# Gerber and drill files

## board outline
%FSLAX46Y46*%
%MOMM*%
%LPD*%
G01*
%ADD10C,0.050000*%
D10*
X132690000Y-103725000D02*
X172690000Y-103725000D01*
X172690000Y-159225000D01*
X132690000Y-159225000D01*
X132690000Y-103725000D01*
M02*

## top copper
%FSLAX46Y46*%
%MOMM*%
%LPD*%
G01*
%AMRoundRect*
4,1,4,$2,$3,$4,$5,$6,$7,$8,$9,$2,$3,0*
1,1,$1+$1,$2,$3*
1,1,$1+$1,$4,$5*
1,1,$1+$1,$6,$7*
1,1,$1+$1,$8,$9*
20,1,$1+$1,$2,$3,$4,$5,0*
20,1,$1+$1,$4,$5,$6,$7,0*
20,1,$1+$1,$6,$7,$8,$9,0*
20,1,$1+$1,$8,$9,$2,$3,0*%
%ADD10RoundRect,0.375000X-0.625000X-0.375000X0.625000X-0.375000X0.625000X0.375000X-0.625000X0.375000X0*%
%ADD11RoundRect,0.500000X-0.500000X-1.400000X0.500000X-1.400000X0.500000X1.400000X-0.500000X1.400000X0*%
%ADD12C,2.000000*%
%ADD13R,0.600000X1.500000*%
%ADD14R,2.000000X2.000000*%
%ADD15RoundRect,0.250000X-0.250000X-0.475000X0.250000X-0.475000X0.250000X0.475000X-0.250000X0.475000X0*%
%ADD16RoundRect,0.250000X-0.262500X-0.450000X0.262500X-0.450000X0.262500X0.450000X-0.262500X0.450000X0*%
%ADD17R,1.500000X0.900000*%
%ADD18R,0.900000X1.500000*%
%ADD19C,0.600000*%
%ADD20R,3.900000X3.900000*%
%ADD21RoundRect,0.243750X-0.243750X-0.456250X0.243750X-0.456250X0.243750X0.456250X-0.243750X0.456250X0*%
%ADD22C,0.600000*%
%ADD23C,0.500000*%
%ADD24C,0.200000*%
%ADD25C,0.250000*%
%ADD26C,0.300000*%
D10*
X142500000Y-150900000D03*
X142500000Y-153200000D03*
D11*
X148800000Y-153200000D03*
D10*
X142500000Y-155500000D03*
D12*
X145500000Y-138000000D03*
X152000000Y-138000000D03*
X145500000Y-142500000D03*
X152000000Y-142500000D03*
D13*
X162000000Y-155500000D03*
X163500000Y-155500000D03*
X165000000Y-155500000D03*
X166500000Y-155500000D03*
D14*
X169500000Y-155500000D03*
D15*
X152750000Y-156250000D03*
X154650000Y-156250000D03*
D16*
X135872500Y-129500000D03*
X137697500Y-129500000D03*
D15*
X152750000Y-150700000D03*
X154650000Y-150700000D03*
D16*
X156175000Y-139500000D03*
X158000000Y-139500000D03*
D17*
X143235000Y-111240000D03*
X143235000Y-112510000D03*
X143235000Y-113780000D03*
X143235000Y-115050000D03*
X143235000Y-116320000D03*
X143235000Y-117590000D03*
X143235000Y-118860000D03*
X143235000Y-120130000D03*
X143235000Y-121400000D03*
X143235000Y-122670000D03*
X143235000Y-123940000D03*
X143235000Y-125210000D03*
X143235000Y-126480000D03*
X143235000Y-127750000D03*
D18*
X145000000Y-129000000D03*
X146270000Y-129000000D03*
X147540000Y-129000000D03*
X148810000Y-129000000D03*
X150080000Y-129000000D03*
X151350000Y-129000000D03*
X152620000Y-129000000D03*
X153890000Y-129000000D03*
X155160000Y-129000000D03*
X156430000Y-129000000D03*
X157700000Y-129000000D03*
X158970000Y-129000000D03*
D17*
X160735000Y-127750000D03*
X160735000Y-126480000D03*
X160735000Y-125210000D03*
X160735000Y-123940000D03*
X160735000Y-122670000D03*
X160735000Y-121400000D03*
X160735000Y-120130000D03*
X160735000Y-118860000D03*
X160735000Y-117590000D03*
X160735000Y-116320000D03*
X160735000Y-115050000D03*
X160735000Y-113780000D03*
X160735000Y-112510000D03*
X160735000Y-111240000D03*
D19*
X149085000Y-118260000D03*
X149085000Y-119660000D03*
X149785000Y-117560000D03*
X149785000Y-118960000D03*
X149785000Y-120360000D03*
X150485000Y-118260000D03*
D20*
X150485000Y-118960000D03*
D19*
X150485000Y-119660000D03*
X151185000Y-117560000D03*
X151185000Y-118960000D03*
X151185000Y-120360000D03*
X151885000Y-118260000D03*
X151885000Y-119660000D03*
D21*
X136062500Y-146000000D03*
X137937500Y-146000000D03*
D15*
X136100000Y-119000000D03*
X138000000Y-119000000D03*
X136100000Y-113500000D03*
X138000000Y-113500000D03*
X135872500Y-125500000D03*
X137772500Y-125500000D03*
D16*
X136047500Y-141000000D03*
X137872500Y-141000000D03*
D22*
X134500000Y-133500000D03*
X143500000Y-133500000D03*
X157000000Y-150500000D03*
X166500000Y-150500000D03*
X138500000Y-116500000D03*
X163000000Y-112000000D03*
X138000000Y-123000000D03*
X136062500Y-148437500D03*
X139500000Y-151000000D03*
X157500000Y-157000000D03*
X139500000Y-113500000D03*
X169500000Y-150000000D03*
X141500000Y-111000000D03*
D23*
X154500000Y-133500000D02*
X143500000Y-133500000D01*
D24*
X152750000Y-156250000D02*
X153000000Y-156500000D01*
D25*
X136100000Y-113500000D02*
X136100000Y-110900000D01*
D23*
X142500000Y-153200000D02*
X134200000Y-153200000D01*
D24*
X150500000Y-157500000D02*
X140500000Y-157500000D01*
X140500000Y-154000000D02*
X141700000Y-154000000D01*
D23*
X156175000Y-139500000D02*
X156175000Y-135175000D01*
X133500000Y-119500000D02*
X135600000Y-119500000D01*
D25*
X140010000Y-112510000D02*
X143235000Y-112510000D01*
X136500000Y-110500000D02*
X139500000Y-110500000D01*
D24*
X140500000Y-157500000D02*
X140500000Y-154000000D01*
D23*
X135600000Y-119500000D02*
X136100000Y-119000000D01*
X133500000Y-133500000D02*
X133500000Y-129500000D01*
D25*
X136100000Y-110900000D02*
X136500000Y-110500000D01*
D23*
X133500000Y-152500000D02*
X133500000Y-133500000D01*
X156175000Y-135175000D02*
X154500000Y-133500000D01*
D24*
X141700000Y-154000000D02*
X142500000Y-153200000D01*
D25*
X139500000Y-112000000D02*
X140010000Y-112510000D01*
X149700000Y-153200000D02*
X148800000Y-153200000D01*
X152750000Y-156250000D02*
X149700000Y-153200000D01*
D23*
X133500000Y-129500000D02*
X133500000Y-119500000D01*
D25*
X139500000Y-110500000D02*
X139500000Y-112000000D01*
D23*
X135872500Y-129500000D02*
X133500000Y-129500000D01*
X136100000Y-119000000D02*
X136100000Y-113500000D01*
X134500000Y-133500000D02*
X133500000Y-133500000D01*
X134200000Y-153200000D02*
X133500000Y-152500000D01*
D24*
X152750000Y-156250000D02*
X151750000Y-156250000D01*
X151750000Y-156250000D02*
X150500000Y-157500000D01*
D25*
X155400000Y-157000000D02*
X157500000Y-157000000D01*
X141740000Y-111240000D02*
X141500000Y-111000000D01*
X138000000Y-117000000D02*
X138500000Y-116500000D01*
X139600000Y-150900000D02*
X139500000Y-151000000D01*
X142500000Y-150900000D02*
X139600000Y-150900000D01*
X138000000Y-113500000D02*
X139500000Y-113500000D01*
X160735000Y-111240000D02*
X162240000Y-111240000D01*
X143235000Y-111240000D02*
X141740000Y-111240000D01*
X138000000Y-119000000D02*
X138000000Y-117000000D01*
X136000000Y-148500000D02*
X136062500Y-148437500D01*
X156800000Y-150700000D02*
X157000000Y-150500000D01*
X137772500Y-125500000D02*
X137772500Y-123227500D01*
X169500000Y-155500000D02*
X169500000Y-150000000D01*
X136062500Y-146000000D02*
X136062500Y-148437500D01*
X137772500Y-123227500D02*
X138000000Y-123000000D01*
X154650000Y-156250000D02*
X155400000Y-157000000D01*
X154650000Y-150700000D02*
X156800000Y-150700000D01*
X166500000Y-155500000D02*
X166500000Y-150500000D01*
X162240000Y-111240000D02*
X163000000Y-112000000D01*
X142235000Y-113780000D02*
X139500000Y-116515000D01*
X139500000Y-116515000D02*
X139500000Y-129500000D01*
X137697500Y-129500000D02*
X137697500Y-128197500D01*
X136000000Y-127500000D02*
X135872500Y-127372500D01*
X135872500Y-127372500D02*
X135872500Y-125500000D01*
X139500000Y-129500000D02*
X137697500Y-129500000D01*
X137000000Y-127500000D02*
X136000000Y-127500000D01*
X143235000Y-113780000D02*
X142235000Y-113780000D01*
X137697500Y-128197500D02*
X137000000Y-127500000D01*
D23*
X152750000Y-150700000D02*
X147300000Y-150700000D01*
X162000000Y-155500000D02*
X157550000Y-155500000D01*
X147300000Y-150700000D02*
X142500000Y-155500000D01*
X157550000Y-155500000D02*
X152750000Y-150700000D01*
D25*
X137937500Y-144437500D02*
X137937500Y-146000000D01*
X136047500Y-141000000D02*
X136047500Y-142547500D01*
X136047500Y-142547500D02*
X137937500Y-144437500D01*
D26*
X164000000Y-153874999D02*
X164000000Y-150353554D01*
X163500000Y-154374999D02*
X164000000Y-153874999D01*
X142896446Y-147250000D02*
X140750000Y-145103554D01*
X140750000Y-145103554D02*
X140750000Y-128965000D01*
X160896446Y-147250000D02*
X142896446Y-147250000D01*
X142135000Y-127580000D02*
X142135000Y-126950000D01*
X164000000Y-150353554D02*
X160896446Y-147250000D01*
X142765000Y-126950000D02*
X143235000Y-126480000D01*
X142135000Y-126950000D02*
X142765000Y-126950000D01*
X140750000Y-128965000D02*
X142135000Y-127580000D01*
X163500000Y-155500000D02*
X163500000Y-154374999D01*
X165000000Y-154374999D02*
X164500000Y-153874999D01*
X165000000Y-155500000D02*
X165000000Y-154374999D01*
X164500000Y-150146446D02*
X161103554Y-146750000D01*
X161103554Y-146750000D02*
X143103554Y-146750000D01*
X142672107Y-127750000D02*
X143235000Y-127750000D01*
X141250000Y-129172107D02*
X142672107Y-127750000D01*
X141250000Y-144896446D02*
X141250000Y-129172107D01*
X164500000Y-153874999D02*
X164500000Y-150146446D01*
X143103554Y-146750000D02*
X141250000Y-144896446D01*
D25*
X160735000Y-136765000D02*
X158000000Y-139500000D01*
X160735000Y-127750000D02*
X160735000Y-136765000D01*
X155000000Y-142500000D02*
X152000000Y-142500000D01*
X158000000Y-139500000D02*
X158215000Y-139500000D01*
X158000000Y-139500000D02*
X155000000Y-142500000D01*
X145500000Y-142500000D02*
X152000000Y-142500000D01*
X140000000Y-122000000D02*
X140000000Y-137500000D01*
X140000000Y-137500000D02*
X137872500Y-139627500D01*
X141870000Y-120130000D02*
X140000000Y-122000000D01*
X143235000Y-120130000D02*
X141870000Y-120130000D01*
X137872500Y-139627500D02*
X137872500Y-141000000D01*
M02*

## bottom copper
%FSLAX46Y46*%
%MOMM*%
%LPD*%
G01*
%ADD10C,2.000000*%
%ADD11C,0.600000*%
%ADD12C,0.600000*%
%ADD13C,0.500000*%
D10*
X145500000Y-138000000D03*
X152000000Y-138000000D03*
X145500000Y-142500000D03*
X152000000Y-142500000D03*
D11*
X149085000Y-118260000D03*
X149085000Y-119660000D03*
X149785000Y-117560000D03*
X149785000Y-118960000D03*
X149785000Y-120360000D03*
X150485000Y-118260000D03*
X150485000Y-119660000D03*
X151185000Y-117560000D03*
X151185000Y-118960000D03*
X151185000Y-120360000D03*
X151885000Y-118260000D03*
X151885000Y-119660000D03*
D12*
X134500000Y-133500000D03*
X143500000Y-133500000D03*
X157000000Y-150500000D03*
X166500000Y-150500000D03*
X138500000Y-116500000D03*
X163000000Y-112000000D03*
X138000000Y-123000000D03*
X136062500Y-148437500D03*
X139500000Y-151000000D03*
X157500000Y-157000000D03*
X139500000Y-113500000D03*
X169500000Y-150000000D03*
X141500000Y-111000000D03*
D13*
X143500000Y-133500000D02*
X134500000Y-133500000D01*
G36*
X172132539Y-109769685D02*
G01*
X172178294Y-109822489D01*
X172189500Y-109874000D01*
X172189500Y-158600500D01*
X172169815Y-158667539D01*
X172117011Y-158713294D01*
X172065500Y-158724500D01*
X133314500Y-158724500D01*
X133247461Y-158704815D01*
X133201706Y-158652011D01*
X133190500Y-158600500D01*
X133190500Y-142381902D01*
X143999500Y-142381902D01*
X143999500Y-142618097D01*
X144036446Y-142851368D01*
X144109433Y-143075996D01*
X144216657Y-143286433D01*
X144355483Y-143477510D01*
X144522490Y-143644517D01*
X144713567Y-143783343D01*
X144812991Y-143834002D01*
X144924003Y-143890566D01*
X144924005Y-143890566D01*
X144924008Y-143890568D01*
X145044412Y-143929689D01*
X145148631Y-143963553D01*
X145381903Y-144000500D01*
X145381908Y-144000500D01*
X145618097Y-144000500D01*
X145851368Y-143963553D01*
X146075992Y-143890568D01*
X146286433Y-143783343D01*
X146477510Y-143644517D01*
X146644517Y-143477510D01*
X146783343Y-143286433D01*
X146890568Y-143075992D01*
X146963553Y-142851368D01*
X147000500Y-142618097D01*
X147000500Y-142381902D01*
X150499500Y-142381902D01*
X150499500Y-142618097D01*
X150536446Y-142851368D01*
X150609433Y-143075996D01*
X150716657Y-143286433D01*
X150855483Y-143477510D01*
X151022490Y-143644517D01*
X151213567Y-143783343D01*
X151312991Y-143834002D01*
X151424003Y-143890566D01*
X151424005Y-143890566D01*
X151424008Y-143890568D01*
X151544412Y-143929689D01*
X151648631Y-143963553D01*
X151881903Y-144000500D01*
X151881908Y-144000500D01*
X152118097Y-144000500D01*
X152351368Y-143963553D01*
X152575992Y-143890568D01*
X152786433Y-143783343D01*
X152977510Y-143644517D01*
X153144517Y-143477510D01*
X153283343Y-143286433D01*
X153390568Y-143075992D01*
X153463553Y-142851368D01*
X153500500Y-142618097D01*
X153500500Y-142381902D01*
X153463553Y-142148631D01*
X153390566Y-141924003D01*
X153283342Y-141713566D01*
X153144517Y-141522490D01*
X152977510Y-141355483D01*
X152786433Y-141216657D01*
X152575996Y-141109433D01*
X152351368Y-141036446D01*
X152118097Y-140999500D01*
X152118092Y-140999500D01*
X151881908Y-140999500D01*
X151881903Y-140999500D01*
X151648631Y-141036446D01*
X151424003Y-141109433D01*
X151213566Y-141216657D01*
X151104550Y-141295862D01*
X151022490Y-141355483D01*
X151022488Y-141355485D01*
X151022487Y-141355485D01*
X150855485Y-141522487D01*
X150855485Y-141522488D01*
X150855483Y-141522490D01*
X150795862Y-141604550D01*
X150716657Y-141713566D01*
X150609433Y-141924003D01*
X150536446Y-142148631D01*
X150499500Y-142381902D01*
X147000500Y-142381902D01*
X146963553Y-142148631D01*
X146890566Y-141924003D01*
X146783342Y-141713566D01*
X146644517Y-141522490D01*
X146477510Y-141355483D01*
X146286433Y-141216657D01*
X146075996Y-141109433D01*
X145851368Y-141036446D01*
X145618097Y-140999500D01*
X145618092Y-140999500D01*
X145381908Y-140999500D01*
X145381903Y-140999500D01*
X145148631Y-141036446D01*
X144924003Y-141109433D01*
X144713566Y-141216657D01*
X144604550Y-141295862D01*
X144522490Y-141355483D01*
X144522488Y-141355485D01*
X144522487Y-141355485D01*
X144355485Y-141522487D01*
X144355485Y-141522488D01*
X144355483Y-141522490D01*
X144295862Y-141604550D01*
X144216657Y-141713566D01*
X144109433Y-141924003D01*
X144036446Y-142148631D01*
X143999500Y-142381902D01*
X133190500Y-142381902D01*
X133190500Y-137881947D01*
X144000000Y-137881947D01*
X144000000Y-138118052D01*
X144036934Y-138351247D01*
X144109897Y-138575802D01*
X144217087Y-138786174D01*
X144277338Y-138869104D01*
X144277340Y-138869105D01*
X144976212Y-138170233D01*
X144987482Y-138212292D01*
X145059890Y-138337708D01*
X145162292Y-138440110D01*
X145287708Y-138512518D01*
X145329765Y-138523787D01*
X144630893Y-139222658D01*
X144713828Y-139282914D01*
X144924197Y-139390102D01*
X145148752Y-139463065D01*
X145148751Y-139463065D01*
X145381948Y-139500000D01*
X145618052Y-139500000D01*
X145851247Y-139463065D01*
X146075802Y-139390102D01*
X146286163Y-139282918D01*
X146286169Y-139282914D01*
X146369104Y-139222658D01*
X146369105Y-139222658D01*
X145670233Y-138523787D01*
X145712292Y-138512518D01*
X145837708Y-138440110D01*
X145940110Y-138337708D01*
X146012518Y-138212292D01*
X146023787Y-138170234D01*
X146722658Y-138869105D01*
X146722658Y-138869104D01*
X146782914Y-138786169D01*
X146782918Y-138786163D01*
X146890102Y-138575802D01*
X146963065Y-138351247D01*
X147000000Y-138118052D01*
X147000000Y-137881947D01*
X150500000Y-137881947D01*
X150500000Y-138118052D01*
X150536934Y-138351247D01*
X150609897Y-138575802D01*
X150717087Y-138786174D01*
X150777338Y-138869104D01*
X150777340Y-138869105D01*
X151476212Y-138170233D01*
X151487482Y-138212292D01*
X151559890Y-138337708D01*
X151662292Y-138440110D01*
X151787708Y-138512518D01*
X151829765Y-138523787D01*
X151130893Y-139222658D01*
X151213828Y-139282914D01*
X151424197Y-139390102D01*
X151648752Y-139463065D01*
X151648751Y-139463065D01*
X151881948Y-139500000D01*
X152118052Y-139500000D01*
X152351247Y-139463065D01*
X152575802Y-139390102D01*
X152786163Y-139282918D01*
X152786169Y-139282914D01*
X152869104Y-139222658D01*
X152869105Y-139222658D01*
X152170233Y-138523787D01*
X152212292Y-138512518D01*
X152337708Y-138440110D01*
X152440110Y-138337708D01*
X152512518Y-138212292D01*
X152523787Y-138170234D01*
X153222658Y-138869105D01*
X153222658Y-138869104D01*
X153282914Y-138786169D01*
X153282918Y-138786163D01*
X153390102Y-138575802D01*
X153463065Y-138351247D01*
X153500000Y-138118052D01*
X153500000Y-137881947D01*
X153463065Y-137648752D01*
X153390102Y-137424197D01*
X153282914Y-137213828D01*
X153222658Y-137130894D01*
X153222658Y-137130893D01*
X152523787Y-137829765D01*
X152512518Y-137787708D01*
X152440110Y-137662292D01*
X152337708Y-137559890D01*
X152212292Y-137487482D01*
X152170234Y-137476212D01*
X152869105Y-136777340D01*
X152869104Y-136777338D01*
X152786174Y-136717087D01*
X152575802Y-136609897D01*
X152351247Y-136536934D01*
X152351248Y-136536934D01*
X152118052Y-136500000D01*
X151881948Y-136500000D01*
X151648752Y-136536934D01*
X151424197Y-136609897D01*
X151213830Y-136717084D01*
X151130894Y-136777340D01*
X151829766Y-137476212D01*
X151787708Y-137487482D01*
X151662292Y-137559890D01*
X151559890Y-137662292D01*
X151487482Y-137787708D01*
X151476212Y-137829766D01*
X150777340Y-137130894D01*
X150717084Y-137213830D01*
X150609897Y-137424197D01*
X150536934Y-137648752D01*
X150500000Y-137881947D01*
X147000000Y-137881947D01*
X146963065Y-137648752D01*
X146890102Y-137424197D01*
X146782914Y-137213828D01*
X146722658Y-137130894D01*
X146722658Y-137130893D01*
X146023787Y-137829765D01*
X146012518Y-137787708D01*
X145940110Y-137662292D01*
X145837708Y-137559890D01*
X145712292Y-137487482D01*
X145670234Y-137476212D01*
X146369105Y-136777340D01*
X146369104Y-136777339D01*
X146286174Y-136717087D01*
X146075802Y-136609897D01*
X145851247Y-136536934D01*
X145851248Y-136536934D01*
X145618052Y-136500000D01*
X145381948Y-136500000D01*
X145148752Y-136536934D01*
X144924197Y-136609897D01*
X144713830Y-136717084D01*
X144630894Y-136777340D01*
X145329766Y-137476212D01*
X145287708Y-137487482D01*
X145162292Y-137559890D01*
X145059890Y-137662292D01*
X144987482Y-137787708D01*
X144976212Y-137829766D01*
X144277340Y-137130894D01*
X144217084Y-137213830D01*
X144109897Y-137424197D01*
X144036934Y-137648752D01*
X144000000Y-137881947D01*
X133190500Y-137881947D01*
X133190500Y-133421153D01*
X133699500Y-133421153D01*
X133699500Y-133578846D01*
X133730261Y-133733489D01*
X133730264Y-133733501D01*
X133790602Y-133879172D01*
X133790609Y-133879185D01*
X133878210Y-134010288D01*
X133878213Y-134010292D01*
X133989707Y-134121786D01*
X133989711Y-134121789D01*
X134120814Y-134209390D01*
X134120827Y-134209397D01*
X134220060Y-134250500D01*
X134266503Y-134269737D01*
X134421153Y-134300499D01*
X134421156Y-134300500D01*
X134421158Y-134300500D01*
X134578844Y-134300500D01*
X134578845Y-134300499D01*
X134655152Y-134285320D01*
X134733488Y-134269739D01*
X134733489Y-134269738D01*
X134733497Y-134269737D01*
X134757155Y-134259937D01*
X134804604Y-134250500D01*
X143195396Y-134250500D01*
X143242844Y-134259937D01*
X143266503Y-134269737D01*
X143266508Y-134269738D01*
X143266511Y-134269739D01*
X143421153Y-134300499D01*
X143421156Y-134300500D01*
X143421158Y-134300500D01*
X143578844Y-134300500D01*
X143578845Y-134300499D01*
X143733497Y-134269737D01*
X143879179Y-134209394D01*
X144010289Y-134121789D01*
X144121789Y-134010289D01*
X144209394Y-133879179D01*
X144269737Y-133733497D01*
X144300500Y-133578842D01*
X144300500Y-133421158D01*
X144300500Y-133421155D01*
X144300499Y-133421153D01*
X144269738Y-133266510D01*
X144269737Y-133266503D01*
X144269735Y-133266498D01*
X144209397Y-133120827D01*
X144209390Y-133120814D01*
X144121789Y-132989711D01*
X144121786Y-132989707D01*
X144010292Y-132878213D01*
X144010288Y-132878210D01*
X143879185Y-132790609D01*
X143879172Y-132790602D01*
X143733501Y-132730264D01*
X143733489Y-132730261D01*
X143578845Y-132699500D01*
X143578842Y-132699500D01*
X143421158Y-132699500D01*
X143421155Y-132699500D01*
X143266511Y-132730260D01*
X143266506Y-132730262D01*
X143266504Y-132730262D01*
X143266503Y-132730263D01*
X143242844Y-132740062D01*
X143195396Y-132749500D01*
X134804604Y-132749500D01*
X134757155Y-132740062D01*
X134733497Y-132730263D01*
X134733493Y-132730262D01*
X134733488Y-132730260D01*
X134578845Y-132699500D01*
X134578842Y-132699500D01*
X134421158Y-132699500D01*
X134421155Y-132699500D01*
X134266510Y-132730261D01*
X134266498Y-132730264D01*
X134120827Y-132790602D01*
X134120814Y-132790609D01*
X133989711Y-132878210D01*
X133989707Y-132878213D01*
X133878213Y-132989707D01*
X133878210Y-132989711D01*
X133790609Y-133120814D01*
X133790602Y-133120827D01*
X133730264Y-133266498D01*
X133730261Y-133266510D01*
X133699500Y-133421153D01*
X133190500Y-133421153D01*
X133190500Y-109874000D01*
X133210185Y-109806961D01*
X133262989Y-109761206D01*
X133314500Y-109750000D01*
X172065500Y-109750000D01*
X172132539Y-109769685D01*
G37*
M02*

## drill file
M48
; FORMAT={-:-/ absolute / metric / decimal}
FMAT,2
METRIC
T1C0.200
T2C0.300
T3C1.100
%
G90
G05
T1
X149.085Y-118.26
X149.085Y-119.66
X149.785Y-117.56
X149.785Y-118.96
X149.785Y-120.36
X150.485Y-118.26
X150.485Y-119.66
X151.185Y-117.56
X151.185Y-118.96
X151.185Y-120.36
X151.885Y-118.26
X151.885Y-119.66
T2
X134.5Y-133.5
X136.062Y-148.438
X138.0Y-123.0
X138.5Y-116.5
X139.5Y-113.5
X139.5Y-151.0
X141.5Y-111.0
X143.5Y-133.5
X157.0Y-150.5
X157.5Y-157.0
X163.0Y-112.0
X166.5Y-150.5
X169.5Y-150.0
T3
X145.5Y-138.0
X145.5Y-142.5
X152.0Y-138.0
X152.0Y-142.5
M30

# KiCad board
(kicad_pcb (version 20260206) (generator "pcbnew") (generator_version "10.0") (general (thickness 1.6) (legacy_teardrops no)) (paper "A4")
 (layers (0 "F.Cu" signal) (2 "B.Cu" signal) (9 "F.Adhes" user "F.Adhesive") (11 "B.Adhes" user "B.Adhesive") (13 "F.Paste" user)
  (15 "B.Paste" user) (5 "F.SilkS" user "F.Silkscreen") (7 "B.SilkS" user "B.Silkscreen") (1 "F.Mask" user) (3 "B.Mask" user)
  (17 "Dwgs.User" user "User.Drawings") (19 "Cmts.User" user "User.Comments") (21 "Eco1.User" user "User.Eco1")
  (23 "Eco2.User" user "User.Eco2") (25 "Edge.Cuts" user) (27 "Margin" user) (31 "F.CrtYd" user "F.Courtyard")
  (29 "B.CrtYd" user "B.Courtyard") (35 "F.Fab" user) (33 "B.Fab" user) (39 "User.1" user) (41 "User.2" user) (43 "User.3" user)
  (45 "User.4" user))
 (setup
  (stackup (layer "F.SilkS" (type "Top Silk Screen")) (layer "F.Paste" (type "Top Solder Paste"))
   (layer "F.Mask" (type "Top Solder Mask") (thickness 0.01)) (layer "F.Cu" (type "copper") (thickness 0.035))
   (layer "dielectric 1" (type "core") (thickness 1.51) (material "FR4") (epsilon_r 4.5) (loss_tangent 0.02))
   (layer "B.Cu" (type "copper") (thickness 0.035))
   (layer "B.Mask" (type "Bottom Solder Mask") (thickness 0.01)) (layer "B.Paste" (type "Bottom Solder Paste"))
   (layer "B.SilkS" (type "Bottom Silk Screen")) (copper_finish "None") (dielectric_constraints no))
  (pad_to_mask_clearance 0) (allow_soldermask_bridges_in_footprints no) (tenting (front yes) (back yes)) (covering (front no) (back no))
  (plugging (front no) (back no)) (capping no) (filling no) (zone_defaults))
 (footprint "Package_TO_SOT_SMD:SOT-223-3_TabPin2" (layer "F.Cu") (at 145.65 153.2)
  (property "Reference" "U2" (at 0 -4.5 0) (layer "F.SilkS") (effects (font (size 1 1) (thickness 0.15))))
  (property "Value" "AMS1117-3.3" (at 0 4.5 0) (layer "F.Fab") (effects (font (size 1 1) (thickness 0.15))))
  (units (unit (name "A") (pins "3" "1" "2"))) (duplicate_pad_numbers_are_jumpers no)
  (pad "1" smd roundrect (at -3.15 -2.3) (size 2 1.5) (layers "F.Cu" "F.Mask" "F.Paste") (roundrect_rratio 0.25) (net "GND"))
  (pad "2" smd roundrect (at -3.15 0) (size 2 1.5) (layers "F.Cu" "F.Mask" "F.Paste") (roundrect_rratio 0.25) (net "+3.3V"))
  (pad "2" smd roundrect (at 3.15 0) (size 2 3.8) (layers "F.Cu" "F.Mask" "F.Paste") (roundrect_rratio 0.25) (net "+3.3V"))
  (pad "3" smd roundrect (at -3.15 2.3) (size 2 1.5) (layers "F.Cu" "F.Mask" "F.Paste") (roundrect_rratio 0.25) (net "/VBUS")))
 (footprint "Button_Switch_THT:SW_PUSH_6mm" (layer "F.Cu") (at 145.5 138)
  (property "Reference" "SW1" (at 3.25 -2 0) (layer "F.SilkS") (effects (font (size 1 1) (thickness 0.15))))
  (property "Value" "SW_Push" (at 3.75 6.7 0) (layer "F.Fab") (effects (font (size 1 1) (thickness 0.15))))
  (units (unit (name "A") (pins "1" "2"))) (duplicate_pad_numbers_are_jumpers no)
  (pad "1" thru_hole circle (at 0 0 90) (size 2 2) (drill 1.1) (layers "*.Cu" "*.Mask") (remove_unused_layers no) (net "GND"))
  (pad "1" thru_hole circle (at 6.5 0 90) (size 2 2) (drill 1.1) (layers "*.Cu" "*.Mask") (remove_unused_layers no) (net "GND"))
  (pad "2" thru_hole circle (at 0 4.5 90) (size 2 2) (drill 1.1) (layers "*.Cu" "*.Mask") (remove_unused_layers no) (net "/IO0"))
  (pad "2" thru_hole circle (at 6.5 4.5 90) (size 2 2) (drill 1.1) (layers "*.Cu" "*.Mask") (remove_unused_layers no) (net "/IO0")))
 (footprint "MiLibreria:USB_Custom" (layer "F.Cu") (at 165 155.5)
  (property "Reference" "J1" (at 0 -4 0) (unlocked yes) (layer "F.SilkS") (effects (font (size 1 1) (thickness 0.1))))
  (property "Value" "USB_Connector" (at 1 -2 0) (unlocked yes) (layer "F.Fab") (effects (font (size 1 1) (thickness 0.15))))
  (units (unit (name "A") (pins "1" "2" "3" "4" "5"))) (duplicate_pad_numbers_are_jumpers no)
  (pad "1" smd rect (at -3 0) (size 0.6 1.5) (layers "F.Cu" "F.Mask" "F.Paste") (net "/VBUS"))
  (pad "2" smd rect (at -1.5 0) (size 0.6 1.5) (layers "F.Cu" "F.Mask" "F.Paste") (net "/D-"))
  (pad "3" smd rect (at 0 0) (size 0.6 1.5) (layers "F.Cu" "F.Mask" "F.Paste") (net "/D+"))
  (pad "4" smd rect (at 1.5 0) (size 0.6 1.5) (layers "F.Cu" "F.Mask" "F.Paste") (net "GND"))
  (pad "5" smd rect (at 4.5 0) (size 2 2) (layers "F.Cu" "F.Mask" "F.Paste") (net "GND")))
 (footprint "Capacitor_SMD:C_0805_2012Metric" (layer "F.Cu") (at 153.7 156.25)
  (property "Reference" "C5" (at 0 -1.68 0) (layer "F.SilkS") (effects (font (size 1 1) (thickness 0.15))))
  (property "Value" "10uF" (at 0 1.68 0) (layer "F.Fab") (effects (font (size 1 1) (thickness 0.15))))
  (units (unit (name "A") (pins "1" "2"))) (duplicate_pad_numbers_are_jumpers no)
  (pad "1" smd roundrect (at -0.95 0) (size 1 1.45) (layers "F.Cu" "F.Mask" "F.Paste") (roundrect_rratio 0.25) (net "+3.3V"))
  (pad "2" smd roundrect (at 0.95 0) (size 1 1.45) (layers "F.Cu" "F.Mask" "F.Paste") (roundrect_rratio 0.25) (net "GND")))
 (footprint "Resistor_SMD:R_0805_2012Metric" (layer "F.Cu") (at 136.785 129.5)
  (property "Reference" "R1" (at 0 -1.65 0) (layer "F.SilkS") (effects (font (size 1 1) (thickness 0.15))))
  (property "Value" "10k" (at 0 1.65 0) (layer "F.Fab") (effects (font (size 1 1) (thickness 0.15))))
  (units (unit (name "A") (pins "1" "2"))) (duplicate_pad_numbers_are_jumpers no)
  (pad "1" smd roundrect (at -0.9125 0) (size 1.025 1.4) (layers "F.Cu" "F.Mask" "F.Paste") (roundrect_rratio 0.243902) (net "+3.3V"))
  (pad "2" smd roundrect (at 0.9125 0) (size 1.025 1.4) (layers "F.Cu" "F.Mask" "F.Paste") (roundrect_rratio 0.243902) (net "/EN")))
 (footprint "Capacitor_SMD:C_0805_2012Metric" (layer "F.Cu") (at 153.7 150.7)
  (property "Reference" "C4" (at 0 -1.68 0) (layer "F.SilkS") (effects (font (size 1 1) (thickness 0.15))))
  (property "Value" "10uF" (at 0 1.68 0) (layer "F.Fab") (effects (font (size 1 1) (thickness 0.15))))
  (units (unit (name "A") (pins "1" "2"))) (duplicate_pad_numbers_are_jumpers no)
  (pad "1" smd roundrect (at -0.95 0) (size 1 1.45) (layers "F.Cu" "F.Mask" "F.Paste") (roundrect_rratio 0.25) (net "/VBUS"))
  (pad "2" smd roundrect (at 0.95 0) (size 1 1.45) (layers "F.Cu" "F.Mask" "F.Paste") (roundrect_rratio 0.25) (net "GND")))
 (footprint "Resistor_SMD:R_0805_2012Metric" (layer "F.Cu") (at 157.0875 139.5)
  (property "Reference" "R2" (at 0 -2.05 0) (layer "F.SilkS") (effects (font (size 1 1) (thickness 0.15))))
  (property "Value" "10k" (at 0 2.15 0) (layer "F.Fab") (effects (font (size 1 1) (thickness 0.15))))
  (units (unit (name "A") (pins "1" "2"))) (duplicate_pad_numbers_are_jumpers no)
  (pad "1" smd roundrect (at -0.9125 0) (size 1.025 1.4) (layers "F.Cu" "F.Mask" "F.Paste") (roundrect_rratio 0.243902) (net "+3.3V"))
  (pad "2" smd roundrect (at 0.9125 0) (size 1.025 1.4) (layers "F.Cu" "F.Mask" "F.Paste") (roundrect_rratio 0.243902) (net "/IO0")))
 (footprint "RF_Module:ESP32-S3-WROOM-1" (layer "F.Cu") (at 151.985 116.5)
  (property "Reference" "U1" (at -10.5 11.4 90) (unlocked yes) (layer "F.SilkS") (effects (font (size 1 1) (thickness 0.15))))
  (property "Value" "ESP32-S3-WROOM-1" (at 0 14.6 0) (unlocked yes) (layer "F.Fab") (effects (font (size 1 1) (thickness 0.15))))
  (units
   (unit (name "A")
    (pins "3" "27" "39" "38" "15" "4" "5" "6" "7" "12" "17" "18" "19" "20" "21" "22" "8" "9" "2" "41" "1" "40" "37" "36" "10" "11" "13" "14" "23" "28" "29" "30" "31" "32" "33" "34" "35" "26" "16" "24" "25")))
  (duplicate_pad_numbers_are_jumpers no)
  (pad "" smd rect (at -2.9 1.06) (size 0.9 0.9) (layers "F.Paste"))
  (pad "" smd rect (at -2.9 2.46 270) (size 0.9 0.9) (layers "F.Paste"))
  (pad "" smd rect (at -2.9 3.86) (size 0.9 0.9) (layers "F.Paste"))
  (pad "" smd rect (at -1.5 1.06 270) (size 0.9 0.9) (layers "F.Paste"))
  (pad "" smd rect (at -1.5 2.46 270) (size 0.9 0.9) (layers "F.Paste"))
  (pad "" smd rect (at -1.5 3.86 270) (size 0.9 0.9) (layers "F.Paste"))
  (pad "" smd rect (at -0.1 1.06 270) (size 0.9 0.9) (layers "F.Paste"))
  (pad "" smd rect (at -0.1 2.46 270) (size 0.9 0.9) (layers "F.Paste"))
  (pad "" smd rect (at -0.1 3.86 270) (size 0.9 0.9) (layers "F.Paste"))
  (pad "1" smd rect (at -8.75 -5.26) (size 1.5 0.9) (layers "F.Cu" "F.Mask" "F.Paste") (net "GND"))
  (pad "2" smd rect (at -8.75 -3.99) (size 1.5 0.9) (layers "F.Cu" "F.Mask" "F.Paste") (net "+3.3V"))
  (pad "3" smd rect (at -8.75 -2.72) (size 1.5 0.9) (layers "F.Cu" "F.Mask" "F.Paste") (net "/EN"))
  (pad "4" smd rect (at -8.75 -1.45) (size 1.5 0.9) (layers "F.Cu" "F.Mask" "F.Paste") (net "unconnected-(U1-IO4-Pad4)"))
  (pad "5" smd rect (at -8.75 -0.18) (size 1.5 0.9) (layers "F.Cu" "F.Mask" "F.Paste") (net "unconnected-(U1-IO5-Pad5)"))
  (pad "6" smd rect (at -8.75 1.09) (size 1.5 0.9) (layers "F.Cu" "F.Mask" "F.Paste") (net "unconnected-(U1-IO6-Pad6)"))
  (pad "7" smd rect (at -8.75 2.36) (size 1.5 0.9) (layers "F.Cu" "F.Mask" "F.Paste") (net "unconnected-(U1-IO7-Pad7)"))
  (pad "8" smd rect (at -8.75 3.63) (size 1.5 0.9) (layers "F.Cu" "F.Mask" "F.Paste") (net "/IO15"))
  (pad "9" smd rect (at -8.75 4.9) (size 1.5 0.9) (layers "F.Cu" "F.Mask" "F.Paste") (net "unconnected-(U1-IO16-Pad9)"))
  (pad "10" smd rect (at -8.75 6.17) (size 1.5 0.9) (layers "F.Cu" "F.Mask" "F.Paste") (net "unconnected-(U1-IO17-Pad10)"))
  (pad "11" smd rect (at -8.75 7.44) (size 1.5 0.9) (layers "F.Cu" "F.Mask" "F.Paste") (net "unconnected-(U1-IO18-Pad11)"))
  (pad "12" smd rect (at -8.75 8.71) (size 1.5 0.9) (layers "F.Cu" "F.Mask" "F.Paste") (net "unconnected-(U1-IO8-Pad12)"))
  (pad "13" smd rect (at -8.75 9.98) (size 1.5 0.9) (layers "F.Cu" "F.Mask" "F.Paste") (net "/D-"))
  (pad "14" smd rect (at -8.75 11.25 180) (size 1.5 0.9) (layers "F.Cu" "F.Mask" "F.Paste") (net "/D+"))
  (pad "15" smd rect (at -6.985 12.5 270) (size 1.5 0.9) (layers "F.Cu" "F.Mask" "F.Paste") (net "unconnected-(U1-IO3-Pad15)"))
  (pad "16" smd rect (at -5.715 12.5 270) (size 1.5 0.9) (layers "F.Cu" "F.Mask" "F.Paste") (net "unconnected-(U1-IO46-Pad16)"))
  (pad "17" smd rect (at -4.445 12.5 270) (size 1.5 0.9) (layers "F.Cu" "F.Mask" "F.Paste") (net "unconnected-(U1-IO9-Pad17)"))
  (pad "18" smd rect (at -3.175 12.5 270) (size 1.5 0.9) (layers "F.Cu" "F.Mask" "F.Paste") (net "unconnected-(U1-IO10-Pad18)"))
  (pad "19" smd rect (at -1.905 12.5 270) (size 1.5 0.9) (layers "F.Cu" "F.Mask" "F.Paste") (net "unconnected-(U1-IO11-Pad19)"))
  (pad "20" smd rect (at -0.635 12.5 270) (size 1.5 0.9) (layers "F.Cu" "F.Mask" "F.Paste") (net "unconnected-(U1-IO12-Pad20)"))
  (pad "21" smd rect (at 0.635 12.5 270) (size 1.5 0.9) (layers "F.Cu" "F.Mask" "F.Paste") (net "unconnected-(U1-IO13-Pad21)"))
  (pad "22" smd rect (at 1.905 12.5 270) (size 1.5 0.9) (layers "F.Cu" "F.Mask" "F.Paste") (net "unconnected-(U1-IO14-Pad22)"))
  (pad "23" smd rect (at 3.175 12.5 270) (size 1.5 0.9) (layers "F.Cu" "F.Mask" "F.Paste") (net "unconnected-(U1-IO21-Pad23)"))
  (pad "24" smd rect (at 4.445 12.5 270) (size 1.5 0.9) (layers "F.Cu" "F.Mask" "F.Paste") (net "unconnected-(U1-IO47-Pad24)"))
  (pad "25" smd rect (at 5.715 12.5 270) (size 1.5 0.9) (layers "F.Cu" "F.Mask" "F.Paste") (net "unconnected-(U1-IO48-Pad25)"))
  (pad "26" smd rect (at 6.985 12.5 270) (size 1.5 0.9) (layers "F.Cu" "F.Mask" "F.Paste") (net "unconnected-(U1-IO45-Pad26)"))
  (pad "27" smd rect (at 8.75 11.25) (size 1.5 0.9) (layers "F.Cu" "F.Mask" "F.Paste") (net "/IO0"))
  (pad "28" smd rect (at 8.75 9.98) (size 1.5 0.9) (layers "F.Cu" "F.Mask" "F.Paste") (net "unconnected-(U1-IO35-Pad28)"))
  (pad "29" smd rect (at 8.75 8.71) (size 1.5 0.9) (layers "F.Cu" "F.Mask" "F.Paste") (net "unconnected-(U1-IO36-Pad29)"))
  (pad "30" smd rect (at 8.75 7.44) (size 1.5 0.9) (layers "F.Cu" "F.Mask" "F.Paste") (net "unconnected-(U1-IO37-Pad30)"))
  (pad "31" smd rect (at 8.75 6.17) (size 1.5 0.9) (layers "F.Cu" "F.Mask" "F.Paste") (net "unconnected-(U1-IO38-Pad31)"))
  (pad "32" smd rect (at 8.75 4.9) (size 1.5 0.9) (layers "F.Cu" "F.Mask" "F.Paste") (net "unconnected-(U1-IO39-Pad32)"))
  (pad "33" smd rect (at 8.75 3.63) (size 1.5 0.9) (layers "F.Cu" "F.Mask" "F.Paste") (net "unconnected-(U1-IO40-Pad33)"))
  (pad "34" smd rect (at 8.75 2.36) (size 1.5 0.9) (layers "F.Cu" "F.Mask" "F.Paste") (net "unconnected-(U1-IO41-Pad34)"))
  (pad "35" smd rect (at 8.75 1.09) (size 1.5 0.9) (layers "F.Cu" "F.Mask" "F.Paste") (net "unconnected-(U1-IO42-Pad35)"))
  (pad "36" smd rect (at 8.75 -0.18) (size 1.5 0.9) (layers "F.Cu" "F.Mask" "F.Paste") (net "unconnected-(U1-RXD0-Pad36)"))
  (pad "37" smd rect (at 8.75 -1.45) (size 1.5 0.9) (layers "F.Cu" "F.Mask" "F.Paste") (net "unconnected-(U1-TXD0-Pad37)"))
  (pad "38" smd rect (at 8.75 -2.72) (size 1.5 0.9) (layers "F.Cu" "F.Mask" "F.Paste") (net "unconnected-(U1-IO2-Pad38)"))
  (pad "39" smd rect (at 8.75 -3.99) (size 1.5 0.9) (layers "F.Cu" "F.Mask" "F.Paste") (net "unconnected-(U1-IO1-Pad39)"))
  (pad "40" smd rect (at 8.75 -5.26) (size 1.5 0.9) (layers "F.Cu" "F.Mask" "F.Paste") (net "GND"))
  (pad "41" thru_hole circle (at -2.9 1.76 90) (size 0.6 0.6) (drill 0.2) (layers "*.Cu" "F.Mask") (remove_unused_layers no) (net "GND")
   (zone_connect 2))
  (pad "41" thru_hole circle (at -2.9 3.16) (size 0.6 0.6) (drill 0.2) (layers "*.Cu" "F.Mask") (remove_unused_layers no) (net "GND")
   (zone_connect 2))
  (pad "41" thru_hole circle (at -2.2 1.06) (size 0.6 0.6) (drill 0.2) (layers "*.Cu" "F.Mask") (remove_unused_layers no) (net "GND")
   (zone_connect 2))
  (pad "41" thru_hole circle (at -2.2 2.46) (size 0.6 0.6) (drill 0.2) (layers "*.Cu" "F.Mask") (remove_unused_layers no) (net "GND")
   (zone_connect 2))
  (pad "41" thru_hole circle (at -2.2 3.86) (size 0.6 0.6) (drill 0.2) (layers "*.Cu" "F.Mask") (remove_unused_layers no) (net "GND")
   (zone_connect 2))
  (pad "41" thru_hole circle (at -1.5 1.76) (size 0.6 0.6) (drill 0.2) (layers "*.Cu" "F.Mask") (remove_unused_layers no) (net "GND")
   (zone_connect 2))
  (pad "41" smd rect (at -1.5 2.46 270) (size 3.9 3.9) (layers "F.Cu" "F.Mask") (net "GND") (zone_connect 2))
  (pad "41" thru_hole circle (at -1.5 3.16) (size 0.6 0.6) (drill 0.2) (layers "*.Cu" "F.Mask") (remove_unused_layers no) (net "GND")
   (zone_connect 2))
  (pad "41" thru_hole circle (at -0.8 1.06) (size 0.6 0.6) (drill 0.2) (layers "*.Cu" "F.Mask") (remove_unused_layers no) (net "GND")
   (zone_connect 2))
  (pad "41" thru_hole circle (at -0.8 2.46) (size 0.6 0.6) (drill 0.2) (layers "*.Cu" "F.Mask") (remove_unused_layers no) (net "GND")
   (zone_connect 2))
  (pad "41" thru_hole circle (at -0.8 3.86) (size 0.6 0.6) (drill 0.2) (layers "*.Cu" "F.Mask") (remove_unused_layers no) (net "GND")
   (zone_connect 2))
  (pad "41" thru_hole circle (at -0.1 1.76) (size 0.6 0.6) (drill 0.2) (layers "*.Cu" "F.Mask") (remove_unused_layers no) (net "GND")
   (zone_connect 2))
  (pad "41" thru_hole circle (at -0.1 3.16) (size 0.6 0.6) (drill 0.2) (layers "*.Cu" "F.Mask") (remove_unused_layers no) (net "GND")
   (zone_connect 2))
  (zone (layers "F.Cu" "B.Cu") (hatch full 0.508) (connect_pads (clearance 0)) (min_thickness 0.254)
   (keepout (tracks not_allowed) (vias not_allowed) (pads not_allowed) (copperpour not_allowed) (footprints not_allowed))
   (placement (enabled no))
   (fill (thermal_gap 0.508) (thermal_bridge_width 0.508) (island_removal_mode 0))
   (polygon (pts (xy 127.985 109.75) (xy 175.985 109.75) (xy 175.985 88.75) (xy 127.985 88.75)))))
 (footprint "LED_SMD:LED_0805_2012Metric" (layer "F.Cu") (at 137 146)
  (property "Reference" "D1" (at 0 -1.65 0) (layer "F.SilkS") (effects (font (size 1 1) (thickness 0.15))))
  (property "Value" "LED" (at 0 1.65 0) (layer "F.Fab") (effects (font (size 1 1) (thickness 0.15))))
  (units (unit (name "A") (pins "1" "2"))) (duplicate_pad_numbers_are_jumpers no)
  (pad "1" smd roundrect (at -0.9375 0) (size 0.975 1.4) (layers "F.Cu" "F.Mask" "F.Paste") (roundrect_rratio 0.25) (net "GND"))
  (pad "2" smd roundrect (at 0.9375 0) (size 0.975 1.4) (layers "F.Cu" "F.Mask" "F.Paste") (roundrect_rratio 0.25) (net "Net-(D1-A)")))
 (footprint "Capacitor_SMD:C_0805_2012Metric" (layer "F.Cu") (at 137.05 119)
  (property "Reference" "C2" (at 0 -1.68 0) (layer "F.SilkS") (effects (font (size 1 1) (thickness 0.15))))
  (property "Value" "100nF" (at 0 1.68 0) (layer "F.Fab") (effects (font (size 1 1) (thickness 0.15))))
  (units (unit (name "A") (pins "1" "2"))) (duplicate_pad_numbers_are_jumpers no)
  (pad "1" smd roundrect (at -0.95 0) (size 1 1.45) (layers "F.Cu" "F.Mask" "F.Paste") (roundrect_rratio 0.25) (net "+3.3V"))
  (pad "2" smd roundrect (at 0.95 0) (size 1 1.45) (layers "F.Cu" "F.Mask" "F.Paste") (roundrect_rratio 0.25) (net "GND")))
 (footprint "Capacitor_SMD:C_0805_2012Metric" (layer "F.Cu") (at 137.05 113.5)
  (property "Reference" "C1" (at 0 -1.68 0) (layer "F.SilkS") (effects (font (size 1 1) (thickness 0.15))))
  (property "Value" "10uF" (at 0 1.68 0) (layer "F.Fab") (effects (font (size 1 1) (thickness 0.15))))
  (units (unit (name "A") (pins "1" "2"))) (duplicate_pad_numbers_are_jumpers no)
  (pad "1" smd roundrect (at -0.95 0) (size 1 1.45) (layers "F.Cu" "F.Mask" "F.Paste") (roundrect_rratio 0.25) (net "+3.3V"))
  (pad "2" smd roundrect (at 0.95 0) (size 1 1.45) (layers "F.Cu" "F.Mask" "F.Paste") (roundrect_rratio 0.25) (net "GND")))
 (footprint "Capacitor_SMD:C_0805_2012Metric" (layer "F.Cu") (at 136.8225 125.5)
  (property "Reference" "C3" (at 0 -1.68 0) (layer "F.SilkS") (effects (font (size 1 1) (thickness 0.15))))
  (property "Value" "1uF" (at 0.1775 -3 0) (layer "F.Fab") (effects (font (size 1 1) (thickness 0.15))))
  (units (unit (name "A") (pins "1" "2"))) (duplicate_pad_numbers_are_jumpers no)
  (pad "1" smd roundrect (at -0.95 0) (size 1 1.45) (layers "F.Cu" "F.Mask" "F.Paste") (roundrect_rratio 0.25) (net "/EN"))
  (pad "2" smd roundrect (at 0.95 0) (size 1 1.45) (layers "F.Cu" "F.Mask" "F.Paste") (roundrect_rratio 0.25) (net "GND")))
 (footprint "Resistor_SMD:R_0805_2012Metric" (layer "F.Cu") (at 136.96 141)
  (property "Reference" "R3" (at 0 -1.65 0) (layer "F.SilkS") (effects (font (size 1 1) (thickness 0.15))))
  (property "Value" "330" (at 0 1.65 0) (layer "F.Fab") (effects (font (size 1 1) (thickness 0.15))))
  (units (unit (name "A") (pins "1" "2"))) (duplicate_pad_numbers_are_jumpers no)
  (pad "1" smd roundrect (at -0.9125 0) (size 1.025 1.4) (layers "F.Cu" "F.Mask" "F.Paste") (roundrect_rratio 0.243902) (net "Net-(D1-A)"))
  (pad "2" smd roundrect (at 0.9125 0) (size 1.025 1.4) (layers "F.Cu" "F.Mask" "F.Paste") (roundrect_rratio 0.243902) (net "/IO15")))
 (gr_rect (start 132.69 103.725) (end 172.69 159.225) (stroke (width 0.05) (type default)) (fill no) (layer "Edge.Cuts"))
 (segment (start 154.5 133.5) (end 143.5 133.5) (width 0.5) (layer "F.Cu") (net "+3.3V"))
 (segment (start 152.75 156.25) (end 153 156.5) (width 0.2) (layer "F.Cu") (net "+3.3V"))
 (segment (start 136.1 113.5) (end 136.1 110.9) (width 0.25) (layer "F.Cu") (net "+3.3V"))
 (segment (start 142.5 153.2) (end 134.2 153.2) (width 0.5) (layer "F.Cu") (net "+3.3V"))
 (segment (start 150.5 157.5) (end 140.5 157.5) (width 0.2) (layer "F.Cu") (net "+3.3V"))
 (segment (start 140.5 154) (end 141.7 154) (width 0.2) (layer "F.Cu") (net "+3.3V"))
 (segment (start 156.175 139.5) (end 156.175 135.175) (width 0.5) (layer "F.Cu") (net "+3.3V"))
 (segment (start 133.5 119.5) (end 135.6 119.5) (width 0.5) (layer "F.Cu") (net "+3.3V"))
 (segment (start 140.01 112.51) (end 143.235 112.51) (width 0.25) (layer "F.Cu") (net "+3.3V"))
 (segment (start 136.5 110.5) (end 139.5 110.5) (width 0.25) (layer "F.Cu") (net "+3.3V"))
 (segment (start 140.5 157.5) (end 140.5 154) (width 0.2) (layer "F.Cu") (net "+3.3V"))
 (segment (start 135.6 119.5) (end 136.1 119) (width 0.5) (layer "F.Cu") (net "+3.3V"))
 (segment (start 133.5 133.5) (end 133.5 129.5) (width 0.5) (layer "F.Cu") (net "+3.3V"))
 (segment (start 136.1 110.9) (end 136.5 110.5) (width 0.25) (layer "F.Cu") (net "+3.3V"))
 (segment (start 133.5 152.5) (end 133.5 133.5) (width 0.5) (layer "F.Cu") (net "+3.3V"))
 (segment (start 156.175 135.175) (end 154.5 133.5) (width 0.5) (layer "F.Cu") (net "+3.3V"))
 (segment (start 141.7 154) (end 142.5 153.2) (width 0.2) (layer "F.Cu") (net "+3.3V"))
 (segment (start 139.5 112) (end 140.01 112.51) (width 0.25) (layer "F.Cu") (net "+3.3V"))
 (segment (start 149.7 153.2) (end 148.8 153.2) (width 0.25) (layer "F.Cu") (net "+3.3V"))
 (segment (start 152.75 156.25) (end 149.7 153.2) (width 0.25) (layer "F.Cu") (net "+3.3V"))
 (segment (start 133.5 129.5) (end 133.5 119.5) (width 0.5) (layer "F.Cu") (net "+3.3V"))
 (segment (start 139.5 110.5) (end 139.5 112) (width 0.25) (layer "F.Cu") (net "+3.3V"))
 (segment (start 135.8725 129.5) (end 133.5 129.5) (width 0.5) (layer "F.Cu") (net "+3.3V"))
 (segment (start 136.1 119) (end 136.1 113.5) (width 0.5) (layer "F.Cu") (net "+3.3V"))
 (segment (start 134.5 133.5) (end 133.5 133.5) (width 0.5) (layer "F.Cu") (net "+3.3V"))
 (segment (start 134.2 153.2) (end 133.5 152.5) (width 0.5) (layer "F.Cu") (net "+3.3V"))
 (segment (start 152.75 156.25) (end 151.75 156.25) (width 0.2) (layer "F.Cu") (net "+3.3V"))
 (segment (start 151.75 156.25) (end 150.5 157.5) (width 0.2) (layer "F.Cu") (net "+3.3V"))
 (via (at 134.5 133.5) (size 0.6) (drill 0.3) (layers "F.Cu" "B.Cu") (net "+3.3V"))
 (via (at 143.5 133.5) (size 0.6) (drill 0.3) (layers "F.Cu" "B.Cu") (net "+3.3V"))
 (segment (start 143.5 133.5) (end 134.5 133.5) (width 0.5) (layer "B.Cu") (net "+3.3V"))
 (segment (start 155.4 157) (end 157.5 157) (width 0.25) (layer "F.Cu") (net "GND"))
 (segment (start 141.74 111.24) (end 141.5 111) (width 0.25) (layer "F.Cu") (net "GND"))
 (segment (start 138 117) (end 138.5 116.5) (width 0.25) (layer "F.Cu") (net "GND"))
 (segment (start 139.6 150.9) (end 139.5 151) (width 0.25) (layer "F.Cu") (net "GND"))
 (segment (start 142.5 150.9) (end 139.6 150.9) (width 0.25) (layer "F.Cu") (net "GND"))
 (segment (start 138 113.5) (end 139.5 113.5) (width 0.25) (layer "F.Cu") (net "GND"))
 (segment (start 160.735 111.24) (end 162.24 111.24) (width 0.25) (layer "F.Cu") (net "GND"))
 (segment (start 143.235 111.24) (end 141.74 111.24) (width 0.25) (layer "F.Cu") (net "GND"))
 (segment (start 138 119) (end 138 117) (width 0.25) (layer "F.Cu") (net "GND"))
 (segment (start 136 148.5) (end 136.0625 148.4375) (width 0.25) (layer "F.Cu") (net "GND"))
 (segment (start 156.8 150.7) (end 157 150.5) (width 0.25) (layer "F.Cu") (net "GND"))
 (segment (start 137.7725 125.5) (end 137.7725 123.2275) (width 0.25) (layer "F.Cu") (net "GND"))
 (segment (start 169.5 155.5) (end 169.5 150) (width 0.25) (layer "F.Cu") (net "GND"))
 (segment (start 136.0625 146) (end 136.0625 148.4375) (width 0.25) (layer "F.Cu") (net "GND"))
 (segment (start 137.7725 123.2275) (end 138 123) (width 0.25) (layer "F.Cu") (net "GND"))
 (segment (start 154.65 156.25) (end 155.4 157) (width 0.25) (layer "F.Cu") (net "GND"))
 (segment (start 154.65 150.7) (end 156.8 150.7) (width 0.25) (layer "F.Cu") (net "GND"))
 (segment (start 166.5 155.5) (end 166.5 150.5) (width 0.25) (layer "F.Cu") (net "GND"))
 (segment (start 162.24 111.24) (end 163 112) (width 0.25) (layer "F.Cu") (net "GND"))
 (via (at 157 150.5) (size 0.6) (drill 0.3) (layers "F.Cu" "B.Cu") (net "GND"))
 (via (at 166.5 150.5) (size 0.6) (drill 0.3) (layers "F.Cu" "B.Cu") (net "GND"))
 (via (at 138.5 116.5) (size 0.6) (drill 0.3) (layers "F.Cu" "B.Cu") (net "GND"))
 (via (at 163 112) (size 0.6) (drill 0.3) (layers "F.Cu" "B.Cu") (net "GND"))
 (via (at 138 123) (size 0.6) (drill 0.3) (layers "F.Cu" "B.Cu") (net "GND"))
 (via (at 136.0625 148.4375) (size 0.6) (drill 0.3) (layers "F.Cu" "B.Cu") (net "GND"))
 (via (at 139.5 151) (size 0.6) (drill 0.3) (layers "F.Cu" "B.Cu") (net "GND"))
 (via (at 157.5 157) (size 0.6) (drill 0.3) (layers "F.Cu" "B.Cu") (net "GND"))
 (via (at 139.5 113.5) (size 0.6) (drill 0.3) (layers "F.Cu" "B.Cu") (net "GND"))
 (via (at 169.5 150) (size 0.6) (drill 0.3) (layers "F.Cu" "B.Cu") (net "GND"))
 (via (at 141.5 111) (size 0.6) (drill 0.3) (layers "F.Cu" "B.Cu") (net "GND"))
 (segment (start 142.235 113.78) (end 139.5 116.515) (width 0.25) (layer "F.Cu") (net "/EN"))
 (segment (start 139.5 116.515) (end 139.5 129.5) (width 0.25) (layer "F.Cu") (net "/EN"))
 (segment (start 137.6975 129.5) (end 137.6975 128.1975) (width 0.25) (layer "F.Cu") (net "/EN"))
 (segment (start 136 127.5) (end 135.8725 127.3725) (width 0.25) (layer "F.Cu") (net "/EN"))
 (segment (start 135.8725 127.3725) (end 135.8725 125.5) (width 0.25) (layer "F.Cu") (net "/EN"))
 (segment (start 139.5 129.5) (end 137.6975 129.5) (width 0.25) (layer "F.Cu") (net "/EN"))
 (segment (start 137 127.5) (end 136 127.5) (width 0.25) (layer "F.Cu") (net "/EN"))
 (segment (start 143.235 113.78) (end 142.235 113.78) (width 0.25) (layer "F.Cu") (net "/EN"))
 (segment (start 137.6975 128.1975) (end 137 127.5) (width 0.25) (layer "F.Cu") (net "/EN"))
 (segment (start 152.75 150.7) (end 147.3 150.7) (width 0.5) (layer "F.Cu") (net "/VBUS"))
 (segment (start 162 155.5) (end 157.55 155.5) (width 0.5) (layer "F.Cu") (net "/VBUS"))
 (segment (start 147.3 150.7) (end 142.5 155.5) (width 0.5) (layer "F.Cu") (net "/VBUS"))
 (segment (start 157.55 155.5) (end 152.75 150.7) (width 0.5) (layer "F.Cu") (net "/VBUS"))
 (segment (start 137.9375 144.4375) (end 137.9375 146) (width 0.25) (layer "F.Cu") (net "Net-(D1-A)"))
 (segment (start 136.0475 141) (end 136.0475 142.5475) (width 0.25) (layer "F.Cu") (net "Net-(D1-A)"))
 (segment (start 136.0475 142.5475) (end 137.9375 144.4375) (width 0.25) (layer "F.Cu") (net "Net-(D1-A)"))
 (segment (start 164 153.874999) (end 164 150.353554) (width 0.3) (layer "F.Cu") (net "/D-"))
 (segment (start 163.5 154.374999) (end 164 153.874999) (width 0.3) (layer "F.Cu") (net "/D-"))
 (segment (start 142.896446 147.25) (end 140.75 145.103554) (width 0.3) (layer "F.Cu") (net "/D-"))
 (segment (start 140.75 145.103554) (end 140.75 128.965) (width 0.3) (layer "F.Cu") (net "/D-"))
 (segment (start 160.896446 147.25) (end 142.896446 147.25) (width 0.3) (layer "F.Cu") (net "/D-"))
 (segment (start 142.135 127.58) (end 142.135 126.95) (width 0.3) (layer "F.Cu") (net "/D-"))
 (segment (start 164 150.353554) (end 160.896446 147.25) (width 0.3) (layer "F.Cu") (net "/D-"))
 (segment (start 142.765 126.95) (end 143.235 126.48) (width 0.3) (layer "F.Cu") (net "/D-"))
 (segment (start 142.135 126.95) (end 142.765 126.95) (width 0.3) (layer "F.Cu") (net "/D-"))
 (segment (start 140.75 128.965) (end 142.135 127.58) (width 0.3) (layer "F.Cu") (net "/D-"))
 (segment (start 163.5 155.5) (end 163.5 154.374999) (width 0.3) (layer "F.Cu") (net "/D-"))
 (segment (start 165 154.374999) (end 164.5 153.874999) (width 0.3) (layer "F.Cu") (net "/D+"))
 (segment (start 165 155.5) (end 165 154.374999) (width 0.3) (layer "F.Cu") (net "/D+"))
 (segment (start 164.5 150.146446) (end 161.103554 146.75) (width 0.3) (layer "F.Cu") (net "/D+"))
 (segment (start 161.103554 146.75) (end 143.103554 146.75) (width 0.3) (layer "F.Cu") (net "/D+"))
 (segment (start 142.672107 127.75) (end 143.235 127.75) (width 0.3) (layer "F.Cu") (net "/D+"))
 (segment (start 141.25 129.172107) (end 142.672107 127.75) (width 0.3) (layer "F.Cu") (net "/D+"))
 (segment (start 141.25 144.896446) (end 141.25 129.172107) (width 0.3) (layer "F.Cu") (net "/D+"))
 (segment (start 164.5 153.874999) (end 164.5 150.146446) (width 0.3) (layer "F.Cu") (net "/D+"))
 (segment (start 143.103554 146.75) (end 141.25 144.896446) (width 0.3) (layer "F.Cu") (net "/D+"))
 (segment (start 160.735 136.765) (end 158 139.5) (width 0.25) (layer "F.Cu") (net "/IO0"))
 (segment (start 160.735 127.75) (end 160.735 136.765) (width 0.25) (layer "F.Cu") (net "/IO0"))
 (segment (start 155 142.5) (end 152 142.5) (width 0.25) (layer "F.Cu") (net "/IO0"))
 (segment (start 158 139.5) (end 158.215 139.5) (width 0.25) (layer "F.Cu") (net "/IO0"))
 (segment (start 158 139.5) (end 155 142.5) (width 0.25) (layer "F.Cu") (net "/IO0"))
 (segment (start 145.5 142.5) (end 152 142.5) (width 0.25) (layer "F.Cu") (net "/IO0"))
 (segment (start 140 122) (end 140 137.5) (width 0.25) (layer "F.Cu") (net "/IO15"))
 (segment (start 140 137.5) (end 137.8725 139.6275) (width 0.25) (layer "F.Cu") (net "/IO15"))
 (segment (start 141.87 120.13) (end 140 122) (width 0.25) (layer "F.Cu") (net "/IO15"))
 (segment (start 143.235 120.13) (end 141.87 120.13) (width 0.25) (layer "F.Cu") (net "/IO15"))
 (segment (start 137.8725 139.6275) (end 137.8725 141) (width 0.25) (layer "F.Cu") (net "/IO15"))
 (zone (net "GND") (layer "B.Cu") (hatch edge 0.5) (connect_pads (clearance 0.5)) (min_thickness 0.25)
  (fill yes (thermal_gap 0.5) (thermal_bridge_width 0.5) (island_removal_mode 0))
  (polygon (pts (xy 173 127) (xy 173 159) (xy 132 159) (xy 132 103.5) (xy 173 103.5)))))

